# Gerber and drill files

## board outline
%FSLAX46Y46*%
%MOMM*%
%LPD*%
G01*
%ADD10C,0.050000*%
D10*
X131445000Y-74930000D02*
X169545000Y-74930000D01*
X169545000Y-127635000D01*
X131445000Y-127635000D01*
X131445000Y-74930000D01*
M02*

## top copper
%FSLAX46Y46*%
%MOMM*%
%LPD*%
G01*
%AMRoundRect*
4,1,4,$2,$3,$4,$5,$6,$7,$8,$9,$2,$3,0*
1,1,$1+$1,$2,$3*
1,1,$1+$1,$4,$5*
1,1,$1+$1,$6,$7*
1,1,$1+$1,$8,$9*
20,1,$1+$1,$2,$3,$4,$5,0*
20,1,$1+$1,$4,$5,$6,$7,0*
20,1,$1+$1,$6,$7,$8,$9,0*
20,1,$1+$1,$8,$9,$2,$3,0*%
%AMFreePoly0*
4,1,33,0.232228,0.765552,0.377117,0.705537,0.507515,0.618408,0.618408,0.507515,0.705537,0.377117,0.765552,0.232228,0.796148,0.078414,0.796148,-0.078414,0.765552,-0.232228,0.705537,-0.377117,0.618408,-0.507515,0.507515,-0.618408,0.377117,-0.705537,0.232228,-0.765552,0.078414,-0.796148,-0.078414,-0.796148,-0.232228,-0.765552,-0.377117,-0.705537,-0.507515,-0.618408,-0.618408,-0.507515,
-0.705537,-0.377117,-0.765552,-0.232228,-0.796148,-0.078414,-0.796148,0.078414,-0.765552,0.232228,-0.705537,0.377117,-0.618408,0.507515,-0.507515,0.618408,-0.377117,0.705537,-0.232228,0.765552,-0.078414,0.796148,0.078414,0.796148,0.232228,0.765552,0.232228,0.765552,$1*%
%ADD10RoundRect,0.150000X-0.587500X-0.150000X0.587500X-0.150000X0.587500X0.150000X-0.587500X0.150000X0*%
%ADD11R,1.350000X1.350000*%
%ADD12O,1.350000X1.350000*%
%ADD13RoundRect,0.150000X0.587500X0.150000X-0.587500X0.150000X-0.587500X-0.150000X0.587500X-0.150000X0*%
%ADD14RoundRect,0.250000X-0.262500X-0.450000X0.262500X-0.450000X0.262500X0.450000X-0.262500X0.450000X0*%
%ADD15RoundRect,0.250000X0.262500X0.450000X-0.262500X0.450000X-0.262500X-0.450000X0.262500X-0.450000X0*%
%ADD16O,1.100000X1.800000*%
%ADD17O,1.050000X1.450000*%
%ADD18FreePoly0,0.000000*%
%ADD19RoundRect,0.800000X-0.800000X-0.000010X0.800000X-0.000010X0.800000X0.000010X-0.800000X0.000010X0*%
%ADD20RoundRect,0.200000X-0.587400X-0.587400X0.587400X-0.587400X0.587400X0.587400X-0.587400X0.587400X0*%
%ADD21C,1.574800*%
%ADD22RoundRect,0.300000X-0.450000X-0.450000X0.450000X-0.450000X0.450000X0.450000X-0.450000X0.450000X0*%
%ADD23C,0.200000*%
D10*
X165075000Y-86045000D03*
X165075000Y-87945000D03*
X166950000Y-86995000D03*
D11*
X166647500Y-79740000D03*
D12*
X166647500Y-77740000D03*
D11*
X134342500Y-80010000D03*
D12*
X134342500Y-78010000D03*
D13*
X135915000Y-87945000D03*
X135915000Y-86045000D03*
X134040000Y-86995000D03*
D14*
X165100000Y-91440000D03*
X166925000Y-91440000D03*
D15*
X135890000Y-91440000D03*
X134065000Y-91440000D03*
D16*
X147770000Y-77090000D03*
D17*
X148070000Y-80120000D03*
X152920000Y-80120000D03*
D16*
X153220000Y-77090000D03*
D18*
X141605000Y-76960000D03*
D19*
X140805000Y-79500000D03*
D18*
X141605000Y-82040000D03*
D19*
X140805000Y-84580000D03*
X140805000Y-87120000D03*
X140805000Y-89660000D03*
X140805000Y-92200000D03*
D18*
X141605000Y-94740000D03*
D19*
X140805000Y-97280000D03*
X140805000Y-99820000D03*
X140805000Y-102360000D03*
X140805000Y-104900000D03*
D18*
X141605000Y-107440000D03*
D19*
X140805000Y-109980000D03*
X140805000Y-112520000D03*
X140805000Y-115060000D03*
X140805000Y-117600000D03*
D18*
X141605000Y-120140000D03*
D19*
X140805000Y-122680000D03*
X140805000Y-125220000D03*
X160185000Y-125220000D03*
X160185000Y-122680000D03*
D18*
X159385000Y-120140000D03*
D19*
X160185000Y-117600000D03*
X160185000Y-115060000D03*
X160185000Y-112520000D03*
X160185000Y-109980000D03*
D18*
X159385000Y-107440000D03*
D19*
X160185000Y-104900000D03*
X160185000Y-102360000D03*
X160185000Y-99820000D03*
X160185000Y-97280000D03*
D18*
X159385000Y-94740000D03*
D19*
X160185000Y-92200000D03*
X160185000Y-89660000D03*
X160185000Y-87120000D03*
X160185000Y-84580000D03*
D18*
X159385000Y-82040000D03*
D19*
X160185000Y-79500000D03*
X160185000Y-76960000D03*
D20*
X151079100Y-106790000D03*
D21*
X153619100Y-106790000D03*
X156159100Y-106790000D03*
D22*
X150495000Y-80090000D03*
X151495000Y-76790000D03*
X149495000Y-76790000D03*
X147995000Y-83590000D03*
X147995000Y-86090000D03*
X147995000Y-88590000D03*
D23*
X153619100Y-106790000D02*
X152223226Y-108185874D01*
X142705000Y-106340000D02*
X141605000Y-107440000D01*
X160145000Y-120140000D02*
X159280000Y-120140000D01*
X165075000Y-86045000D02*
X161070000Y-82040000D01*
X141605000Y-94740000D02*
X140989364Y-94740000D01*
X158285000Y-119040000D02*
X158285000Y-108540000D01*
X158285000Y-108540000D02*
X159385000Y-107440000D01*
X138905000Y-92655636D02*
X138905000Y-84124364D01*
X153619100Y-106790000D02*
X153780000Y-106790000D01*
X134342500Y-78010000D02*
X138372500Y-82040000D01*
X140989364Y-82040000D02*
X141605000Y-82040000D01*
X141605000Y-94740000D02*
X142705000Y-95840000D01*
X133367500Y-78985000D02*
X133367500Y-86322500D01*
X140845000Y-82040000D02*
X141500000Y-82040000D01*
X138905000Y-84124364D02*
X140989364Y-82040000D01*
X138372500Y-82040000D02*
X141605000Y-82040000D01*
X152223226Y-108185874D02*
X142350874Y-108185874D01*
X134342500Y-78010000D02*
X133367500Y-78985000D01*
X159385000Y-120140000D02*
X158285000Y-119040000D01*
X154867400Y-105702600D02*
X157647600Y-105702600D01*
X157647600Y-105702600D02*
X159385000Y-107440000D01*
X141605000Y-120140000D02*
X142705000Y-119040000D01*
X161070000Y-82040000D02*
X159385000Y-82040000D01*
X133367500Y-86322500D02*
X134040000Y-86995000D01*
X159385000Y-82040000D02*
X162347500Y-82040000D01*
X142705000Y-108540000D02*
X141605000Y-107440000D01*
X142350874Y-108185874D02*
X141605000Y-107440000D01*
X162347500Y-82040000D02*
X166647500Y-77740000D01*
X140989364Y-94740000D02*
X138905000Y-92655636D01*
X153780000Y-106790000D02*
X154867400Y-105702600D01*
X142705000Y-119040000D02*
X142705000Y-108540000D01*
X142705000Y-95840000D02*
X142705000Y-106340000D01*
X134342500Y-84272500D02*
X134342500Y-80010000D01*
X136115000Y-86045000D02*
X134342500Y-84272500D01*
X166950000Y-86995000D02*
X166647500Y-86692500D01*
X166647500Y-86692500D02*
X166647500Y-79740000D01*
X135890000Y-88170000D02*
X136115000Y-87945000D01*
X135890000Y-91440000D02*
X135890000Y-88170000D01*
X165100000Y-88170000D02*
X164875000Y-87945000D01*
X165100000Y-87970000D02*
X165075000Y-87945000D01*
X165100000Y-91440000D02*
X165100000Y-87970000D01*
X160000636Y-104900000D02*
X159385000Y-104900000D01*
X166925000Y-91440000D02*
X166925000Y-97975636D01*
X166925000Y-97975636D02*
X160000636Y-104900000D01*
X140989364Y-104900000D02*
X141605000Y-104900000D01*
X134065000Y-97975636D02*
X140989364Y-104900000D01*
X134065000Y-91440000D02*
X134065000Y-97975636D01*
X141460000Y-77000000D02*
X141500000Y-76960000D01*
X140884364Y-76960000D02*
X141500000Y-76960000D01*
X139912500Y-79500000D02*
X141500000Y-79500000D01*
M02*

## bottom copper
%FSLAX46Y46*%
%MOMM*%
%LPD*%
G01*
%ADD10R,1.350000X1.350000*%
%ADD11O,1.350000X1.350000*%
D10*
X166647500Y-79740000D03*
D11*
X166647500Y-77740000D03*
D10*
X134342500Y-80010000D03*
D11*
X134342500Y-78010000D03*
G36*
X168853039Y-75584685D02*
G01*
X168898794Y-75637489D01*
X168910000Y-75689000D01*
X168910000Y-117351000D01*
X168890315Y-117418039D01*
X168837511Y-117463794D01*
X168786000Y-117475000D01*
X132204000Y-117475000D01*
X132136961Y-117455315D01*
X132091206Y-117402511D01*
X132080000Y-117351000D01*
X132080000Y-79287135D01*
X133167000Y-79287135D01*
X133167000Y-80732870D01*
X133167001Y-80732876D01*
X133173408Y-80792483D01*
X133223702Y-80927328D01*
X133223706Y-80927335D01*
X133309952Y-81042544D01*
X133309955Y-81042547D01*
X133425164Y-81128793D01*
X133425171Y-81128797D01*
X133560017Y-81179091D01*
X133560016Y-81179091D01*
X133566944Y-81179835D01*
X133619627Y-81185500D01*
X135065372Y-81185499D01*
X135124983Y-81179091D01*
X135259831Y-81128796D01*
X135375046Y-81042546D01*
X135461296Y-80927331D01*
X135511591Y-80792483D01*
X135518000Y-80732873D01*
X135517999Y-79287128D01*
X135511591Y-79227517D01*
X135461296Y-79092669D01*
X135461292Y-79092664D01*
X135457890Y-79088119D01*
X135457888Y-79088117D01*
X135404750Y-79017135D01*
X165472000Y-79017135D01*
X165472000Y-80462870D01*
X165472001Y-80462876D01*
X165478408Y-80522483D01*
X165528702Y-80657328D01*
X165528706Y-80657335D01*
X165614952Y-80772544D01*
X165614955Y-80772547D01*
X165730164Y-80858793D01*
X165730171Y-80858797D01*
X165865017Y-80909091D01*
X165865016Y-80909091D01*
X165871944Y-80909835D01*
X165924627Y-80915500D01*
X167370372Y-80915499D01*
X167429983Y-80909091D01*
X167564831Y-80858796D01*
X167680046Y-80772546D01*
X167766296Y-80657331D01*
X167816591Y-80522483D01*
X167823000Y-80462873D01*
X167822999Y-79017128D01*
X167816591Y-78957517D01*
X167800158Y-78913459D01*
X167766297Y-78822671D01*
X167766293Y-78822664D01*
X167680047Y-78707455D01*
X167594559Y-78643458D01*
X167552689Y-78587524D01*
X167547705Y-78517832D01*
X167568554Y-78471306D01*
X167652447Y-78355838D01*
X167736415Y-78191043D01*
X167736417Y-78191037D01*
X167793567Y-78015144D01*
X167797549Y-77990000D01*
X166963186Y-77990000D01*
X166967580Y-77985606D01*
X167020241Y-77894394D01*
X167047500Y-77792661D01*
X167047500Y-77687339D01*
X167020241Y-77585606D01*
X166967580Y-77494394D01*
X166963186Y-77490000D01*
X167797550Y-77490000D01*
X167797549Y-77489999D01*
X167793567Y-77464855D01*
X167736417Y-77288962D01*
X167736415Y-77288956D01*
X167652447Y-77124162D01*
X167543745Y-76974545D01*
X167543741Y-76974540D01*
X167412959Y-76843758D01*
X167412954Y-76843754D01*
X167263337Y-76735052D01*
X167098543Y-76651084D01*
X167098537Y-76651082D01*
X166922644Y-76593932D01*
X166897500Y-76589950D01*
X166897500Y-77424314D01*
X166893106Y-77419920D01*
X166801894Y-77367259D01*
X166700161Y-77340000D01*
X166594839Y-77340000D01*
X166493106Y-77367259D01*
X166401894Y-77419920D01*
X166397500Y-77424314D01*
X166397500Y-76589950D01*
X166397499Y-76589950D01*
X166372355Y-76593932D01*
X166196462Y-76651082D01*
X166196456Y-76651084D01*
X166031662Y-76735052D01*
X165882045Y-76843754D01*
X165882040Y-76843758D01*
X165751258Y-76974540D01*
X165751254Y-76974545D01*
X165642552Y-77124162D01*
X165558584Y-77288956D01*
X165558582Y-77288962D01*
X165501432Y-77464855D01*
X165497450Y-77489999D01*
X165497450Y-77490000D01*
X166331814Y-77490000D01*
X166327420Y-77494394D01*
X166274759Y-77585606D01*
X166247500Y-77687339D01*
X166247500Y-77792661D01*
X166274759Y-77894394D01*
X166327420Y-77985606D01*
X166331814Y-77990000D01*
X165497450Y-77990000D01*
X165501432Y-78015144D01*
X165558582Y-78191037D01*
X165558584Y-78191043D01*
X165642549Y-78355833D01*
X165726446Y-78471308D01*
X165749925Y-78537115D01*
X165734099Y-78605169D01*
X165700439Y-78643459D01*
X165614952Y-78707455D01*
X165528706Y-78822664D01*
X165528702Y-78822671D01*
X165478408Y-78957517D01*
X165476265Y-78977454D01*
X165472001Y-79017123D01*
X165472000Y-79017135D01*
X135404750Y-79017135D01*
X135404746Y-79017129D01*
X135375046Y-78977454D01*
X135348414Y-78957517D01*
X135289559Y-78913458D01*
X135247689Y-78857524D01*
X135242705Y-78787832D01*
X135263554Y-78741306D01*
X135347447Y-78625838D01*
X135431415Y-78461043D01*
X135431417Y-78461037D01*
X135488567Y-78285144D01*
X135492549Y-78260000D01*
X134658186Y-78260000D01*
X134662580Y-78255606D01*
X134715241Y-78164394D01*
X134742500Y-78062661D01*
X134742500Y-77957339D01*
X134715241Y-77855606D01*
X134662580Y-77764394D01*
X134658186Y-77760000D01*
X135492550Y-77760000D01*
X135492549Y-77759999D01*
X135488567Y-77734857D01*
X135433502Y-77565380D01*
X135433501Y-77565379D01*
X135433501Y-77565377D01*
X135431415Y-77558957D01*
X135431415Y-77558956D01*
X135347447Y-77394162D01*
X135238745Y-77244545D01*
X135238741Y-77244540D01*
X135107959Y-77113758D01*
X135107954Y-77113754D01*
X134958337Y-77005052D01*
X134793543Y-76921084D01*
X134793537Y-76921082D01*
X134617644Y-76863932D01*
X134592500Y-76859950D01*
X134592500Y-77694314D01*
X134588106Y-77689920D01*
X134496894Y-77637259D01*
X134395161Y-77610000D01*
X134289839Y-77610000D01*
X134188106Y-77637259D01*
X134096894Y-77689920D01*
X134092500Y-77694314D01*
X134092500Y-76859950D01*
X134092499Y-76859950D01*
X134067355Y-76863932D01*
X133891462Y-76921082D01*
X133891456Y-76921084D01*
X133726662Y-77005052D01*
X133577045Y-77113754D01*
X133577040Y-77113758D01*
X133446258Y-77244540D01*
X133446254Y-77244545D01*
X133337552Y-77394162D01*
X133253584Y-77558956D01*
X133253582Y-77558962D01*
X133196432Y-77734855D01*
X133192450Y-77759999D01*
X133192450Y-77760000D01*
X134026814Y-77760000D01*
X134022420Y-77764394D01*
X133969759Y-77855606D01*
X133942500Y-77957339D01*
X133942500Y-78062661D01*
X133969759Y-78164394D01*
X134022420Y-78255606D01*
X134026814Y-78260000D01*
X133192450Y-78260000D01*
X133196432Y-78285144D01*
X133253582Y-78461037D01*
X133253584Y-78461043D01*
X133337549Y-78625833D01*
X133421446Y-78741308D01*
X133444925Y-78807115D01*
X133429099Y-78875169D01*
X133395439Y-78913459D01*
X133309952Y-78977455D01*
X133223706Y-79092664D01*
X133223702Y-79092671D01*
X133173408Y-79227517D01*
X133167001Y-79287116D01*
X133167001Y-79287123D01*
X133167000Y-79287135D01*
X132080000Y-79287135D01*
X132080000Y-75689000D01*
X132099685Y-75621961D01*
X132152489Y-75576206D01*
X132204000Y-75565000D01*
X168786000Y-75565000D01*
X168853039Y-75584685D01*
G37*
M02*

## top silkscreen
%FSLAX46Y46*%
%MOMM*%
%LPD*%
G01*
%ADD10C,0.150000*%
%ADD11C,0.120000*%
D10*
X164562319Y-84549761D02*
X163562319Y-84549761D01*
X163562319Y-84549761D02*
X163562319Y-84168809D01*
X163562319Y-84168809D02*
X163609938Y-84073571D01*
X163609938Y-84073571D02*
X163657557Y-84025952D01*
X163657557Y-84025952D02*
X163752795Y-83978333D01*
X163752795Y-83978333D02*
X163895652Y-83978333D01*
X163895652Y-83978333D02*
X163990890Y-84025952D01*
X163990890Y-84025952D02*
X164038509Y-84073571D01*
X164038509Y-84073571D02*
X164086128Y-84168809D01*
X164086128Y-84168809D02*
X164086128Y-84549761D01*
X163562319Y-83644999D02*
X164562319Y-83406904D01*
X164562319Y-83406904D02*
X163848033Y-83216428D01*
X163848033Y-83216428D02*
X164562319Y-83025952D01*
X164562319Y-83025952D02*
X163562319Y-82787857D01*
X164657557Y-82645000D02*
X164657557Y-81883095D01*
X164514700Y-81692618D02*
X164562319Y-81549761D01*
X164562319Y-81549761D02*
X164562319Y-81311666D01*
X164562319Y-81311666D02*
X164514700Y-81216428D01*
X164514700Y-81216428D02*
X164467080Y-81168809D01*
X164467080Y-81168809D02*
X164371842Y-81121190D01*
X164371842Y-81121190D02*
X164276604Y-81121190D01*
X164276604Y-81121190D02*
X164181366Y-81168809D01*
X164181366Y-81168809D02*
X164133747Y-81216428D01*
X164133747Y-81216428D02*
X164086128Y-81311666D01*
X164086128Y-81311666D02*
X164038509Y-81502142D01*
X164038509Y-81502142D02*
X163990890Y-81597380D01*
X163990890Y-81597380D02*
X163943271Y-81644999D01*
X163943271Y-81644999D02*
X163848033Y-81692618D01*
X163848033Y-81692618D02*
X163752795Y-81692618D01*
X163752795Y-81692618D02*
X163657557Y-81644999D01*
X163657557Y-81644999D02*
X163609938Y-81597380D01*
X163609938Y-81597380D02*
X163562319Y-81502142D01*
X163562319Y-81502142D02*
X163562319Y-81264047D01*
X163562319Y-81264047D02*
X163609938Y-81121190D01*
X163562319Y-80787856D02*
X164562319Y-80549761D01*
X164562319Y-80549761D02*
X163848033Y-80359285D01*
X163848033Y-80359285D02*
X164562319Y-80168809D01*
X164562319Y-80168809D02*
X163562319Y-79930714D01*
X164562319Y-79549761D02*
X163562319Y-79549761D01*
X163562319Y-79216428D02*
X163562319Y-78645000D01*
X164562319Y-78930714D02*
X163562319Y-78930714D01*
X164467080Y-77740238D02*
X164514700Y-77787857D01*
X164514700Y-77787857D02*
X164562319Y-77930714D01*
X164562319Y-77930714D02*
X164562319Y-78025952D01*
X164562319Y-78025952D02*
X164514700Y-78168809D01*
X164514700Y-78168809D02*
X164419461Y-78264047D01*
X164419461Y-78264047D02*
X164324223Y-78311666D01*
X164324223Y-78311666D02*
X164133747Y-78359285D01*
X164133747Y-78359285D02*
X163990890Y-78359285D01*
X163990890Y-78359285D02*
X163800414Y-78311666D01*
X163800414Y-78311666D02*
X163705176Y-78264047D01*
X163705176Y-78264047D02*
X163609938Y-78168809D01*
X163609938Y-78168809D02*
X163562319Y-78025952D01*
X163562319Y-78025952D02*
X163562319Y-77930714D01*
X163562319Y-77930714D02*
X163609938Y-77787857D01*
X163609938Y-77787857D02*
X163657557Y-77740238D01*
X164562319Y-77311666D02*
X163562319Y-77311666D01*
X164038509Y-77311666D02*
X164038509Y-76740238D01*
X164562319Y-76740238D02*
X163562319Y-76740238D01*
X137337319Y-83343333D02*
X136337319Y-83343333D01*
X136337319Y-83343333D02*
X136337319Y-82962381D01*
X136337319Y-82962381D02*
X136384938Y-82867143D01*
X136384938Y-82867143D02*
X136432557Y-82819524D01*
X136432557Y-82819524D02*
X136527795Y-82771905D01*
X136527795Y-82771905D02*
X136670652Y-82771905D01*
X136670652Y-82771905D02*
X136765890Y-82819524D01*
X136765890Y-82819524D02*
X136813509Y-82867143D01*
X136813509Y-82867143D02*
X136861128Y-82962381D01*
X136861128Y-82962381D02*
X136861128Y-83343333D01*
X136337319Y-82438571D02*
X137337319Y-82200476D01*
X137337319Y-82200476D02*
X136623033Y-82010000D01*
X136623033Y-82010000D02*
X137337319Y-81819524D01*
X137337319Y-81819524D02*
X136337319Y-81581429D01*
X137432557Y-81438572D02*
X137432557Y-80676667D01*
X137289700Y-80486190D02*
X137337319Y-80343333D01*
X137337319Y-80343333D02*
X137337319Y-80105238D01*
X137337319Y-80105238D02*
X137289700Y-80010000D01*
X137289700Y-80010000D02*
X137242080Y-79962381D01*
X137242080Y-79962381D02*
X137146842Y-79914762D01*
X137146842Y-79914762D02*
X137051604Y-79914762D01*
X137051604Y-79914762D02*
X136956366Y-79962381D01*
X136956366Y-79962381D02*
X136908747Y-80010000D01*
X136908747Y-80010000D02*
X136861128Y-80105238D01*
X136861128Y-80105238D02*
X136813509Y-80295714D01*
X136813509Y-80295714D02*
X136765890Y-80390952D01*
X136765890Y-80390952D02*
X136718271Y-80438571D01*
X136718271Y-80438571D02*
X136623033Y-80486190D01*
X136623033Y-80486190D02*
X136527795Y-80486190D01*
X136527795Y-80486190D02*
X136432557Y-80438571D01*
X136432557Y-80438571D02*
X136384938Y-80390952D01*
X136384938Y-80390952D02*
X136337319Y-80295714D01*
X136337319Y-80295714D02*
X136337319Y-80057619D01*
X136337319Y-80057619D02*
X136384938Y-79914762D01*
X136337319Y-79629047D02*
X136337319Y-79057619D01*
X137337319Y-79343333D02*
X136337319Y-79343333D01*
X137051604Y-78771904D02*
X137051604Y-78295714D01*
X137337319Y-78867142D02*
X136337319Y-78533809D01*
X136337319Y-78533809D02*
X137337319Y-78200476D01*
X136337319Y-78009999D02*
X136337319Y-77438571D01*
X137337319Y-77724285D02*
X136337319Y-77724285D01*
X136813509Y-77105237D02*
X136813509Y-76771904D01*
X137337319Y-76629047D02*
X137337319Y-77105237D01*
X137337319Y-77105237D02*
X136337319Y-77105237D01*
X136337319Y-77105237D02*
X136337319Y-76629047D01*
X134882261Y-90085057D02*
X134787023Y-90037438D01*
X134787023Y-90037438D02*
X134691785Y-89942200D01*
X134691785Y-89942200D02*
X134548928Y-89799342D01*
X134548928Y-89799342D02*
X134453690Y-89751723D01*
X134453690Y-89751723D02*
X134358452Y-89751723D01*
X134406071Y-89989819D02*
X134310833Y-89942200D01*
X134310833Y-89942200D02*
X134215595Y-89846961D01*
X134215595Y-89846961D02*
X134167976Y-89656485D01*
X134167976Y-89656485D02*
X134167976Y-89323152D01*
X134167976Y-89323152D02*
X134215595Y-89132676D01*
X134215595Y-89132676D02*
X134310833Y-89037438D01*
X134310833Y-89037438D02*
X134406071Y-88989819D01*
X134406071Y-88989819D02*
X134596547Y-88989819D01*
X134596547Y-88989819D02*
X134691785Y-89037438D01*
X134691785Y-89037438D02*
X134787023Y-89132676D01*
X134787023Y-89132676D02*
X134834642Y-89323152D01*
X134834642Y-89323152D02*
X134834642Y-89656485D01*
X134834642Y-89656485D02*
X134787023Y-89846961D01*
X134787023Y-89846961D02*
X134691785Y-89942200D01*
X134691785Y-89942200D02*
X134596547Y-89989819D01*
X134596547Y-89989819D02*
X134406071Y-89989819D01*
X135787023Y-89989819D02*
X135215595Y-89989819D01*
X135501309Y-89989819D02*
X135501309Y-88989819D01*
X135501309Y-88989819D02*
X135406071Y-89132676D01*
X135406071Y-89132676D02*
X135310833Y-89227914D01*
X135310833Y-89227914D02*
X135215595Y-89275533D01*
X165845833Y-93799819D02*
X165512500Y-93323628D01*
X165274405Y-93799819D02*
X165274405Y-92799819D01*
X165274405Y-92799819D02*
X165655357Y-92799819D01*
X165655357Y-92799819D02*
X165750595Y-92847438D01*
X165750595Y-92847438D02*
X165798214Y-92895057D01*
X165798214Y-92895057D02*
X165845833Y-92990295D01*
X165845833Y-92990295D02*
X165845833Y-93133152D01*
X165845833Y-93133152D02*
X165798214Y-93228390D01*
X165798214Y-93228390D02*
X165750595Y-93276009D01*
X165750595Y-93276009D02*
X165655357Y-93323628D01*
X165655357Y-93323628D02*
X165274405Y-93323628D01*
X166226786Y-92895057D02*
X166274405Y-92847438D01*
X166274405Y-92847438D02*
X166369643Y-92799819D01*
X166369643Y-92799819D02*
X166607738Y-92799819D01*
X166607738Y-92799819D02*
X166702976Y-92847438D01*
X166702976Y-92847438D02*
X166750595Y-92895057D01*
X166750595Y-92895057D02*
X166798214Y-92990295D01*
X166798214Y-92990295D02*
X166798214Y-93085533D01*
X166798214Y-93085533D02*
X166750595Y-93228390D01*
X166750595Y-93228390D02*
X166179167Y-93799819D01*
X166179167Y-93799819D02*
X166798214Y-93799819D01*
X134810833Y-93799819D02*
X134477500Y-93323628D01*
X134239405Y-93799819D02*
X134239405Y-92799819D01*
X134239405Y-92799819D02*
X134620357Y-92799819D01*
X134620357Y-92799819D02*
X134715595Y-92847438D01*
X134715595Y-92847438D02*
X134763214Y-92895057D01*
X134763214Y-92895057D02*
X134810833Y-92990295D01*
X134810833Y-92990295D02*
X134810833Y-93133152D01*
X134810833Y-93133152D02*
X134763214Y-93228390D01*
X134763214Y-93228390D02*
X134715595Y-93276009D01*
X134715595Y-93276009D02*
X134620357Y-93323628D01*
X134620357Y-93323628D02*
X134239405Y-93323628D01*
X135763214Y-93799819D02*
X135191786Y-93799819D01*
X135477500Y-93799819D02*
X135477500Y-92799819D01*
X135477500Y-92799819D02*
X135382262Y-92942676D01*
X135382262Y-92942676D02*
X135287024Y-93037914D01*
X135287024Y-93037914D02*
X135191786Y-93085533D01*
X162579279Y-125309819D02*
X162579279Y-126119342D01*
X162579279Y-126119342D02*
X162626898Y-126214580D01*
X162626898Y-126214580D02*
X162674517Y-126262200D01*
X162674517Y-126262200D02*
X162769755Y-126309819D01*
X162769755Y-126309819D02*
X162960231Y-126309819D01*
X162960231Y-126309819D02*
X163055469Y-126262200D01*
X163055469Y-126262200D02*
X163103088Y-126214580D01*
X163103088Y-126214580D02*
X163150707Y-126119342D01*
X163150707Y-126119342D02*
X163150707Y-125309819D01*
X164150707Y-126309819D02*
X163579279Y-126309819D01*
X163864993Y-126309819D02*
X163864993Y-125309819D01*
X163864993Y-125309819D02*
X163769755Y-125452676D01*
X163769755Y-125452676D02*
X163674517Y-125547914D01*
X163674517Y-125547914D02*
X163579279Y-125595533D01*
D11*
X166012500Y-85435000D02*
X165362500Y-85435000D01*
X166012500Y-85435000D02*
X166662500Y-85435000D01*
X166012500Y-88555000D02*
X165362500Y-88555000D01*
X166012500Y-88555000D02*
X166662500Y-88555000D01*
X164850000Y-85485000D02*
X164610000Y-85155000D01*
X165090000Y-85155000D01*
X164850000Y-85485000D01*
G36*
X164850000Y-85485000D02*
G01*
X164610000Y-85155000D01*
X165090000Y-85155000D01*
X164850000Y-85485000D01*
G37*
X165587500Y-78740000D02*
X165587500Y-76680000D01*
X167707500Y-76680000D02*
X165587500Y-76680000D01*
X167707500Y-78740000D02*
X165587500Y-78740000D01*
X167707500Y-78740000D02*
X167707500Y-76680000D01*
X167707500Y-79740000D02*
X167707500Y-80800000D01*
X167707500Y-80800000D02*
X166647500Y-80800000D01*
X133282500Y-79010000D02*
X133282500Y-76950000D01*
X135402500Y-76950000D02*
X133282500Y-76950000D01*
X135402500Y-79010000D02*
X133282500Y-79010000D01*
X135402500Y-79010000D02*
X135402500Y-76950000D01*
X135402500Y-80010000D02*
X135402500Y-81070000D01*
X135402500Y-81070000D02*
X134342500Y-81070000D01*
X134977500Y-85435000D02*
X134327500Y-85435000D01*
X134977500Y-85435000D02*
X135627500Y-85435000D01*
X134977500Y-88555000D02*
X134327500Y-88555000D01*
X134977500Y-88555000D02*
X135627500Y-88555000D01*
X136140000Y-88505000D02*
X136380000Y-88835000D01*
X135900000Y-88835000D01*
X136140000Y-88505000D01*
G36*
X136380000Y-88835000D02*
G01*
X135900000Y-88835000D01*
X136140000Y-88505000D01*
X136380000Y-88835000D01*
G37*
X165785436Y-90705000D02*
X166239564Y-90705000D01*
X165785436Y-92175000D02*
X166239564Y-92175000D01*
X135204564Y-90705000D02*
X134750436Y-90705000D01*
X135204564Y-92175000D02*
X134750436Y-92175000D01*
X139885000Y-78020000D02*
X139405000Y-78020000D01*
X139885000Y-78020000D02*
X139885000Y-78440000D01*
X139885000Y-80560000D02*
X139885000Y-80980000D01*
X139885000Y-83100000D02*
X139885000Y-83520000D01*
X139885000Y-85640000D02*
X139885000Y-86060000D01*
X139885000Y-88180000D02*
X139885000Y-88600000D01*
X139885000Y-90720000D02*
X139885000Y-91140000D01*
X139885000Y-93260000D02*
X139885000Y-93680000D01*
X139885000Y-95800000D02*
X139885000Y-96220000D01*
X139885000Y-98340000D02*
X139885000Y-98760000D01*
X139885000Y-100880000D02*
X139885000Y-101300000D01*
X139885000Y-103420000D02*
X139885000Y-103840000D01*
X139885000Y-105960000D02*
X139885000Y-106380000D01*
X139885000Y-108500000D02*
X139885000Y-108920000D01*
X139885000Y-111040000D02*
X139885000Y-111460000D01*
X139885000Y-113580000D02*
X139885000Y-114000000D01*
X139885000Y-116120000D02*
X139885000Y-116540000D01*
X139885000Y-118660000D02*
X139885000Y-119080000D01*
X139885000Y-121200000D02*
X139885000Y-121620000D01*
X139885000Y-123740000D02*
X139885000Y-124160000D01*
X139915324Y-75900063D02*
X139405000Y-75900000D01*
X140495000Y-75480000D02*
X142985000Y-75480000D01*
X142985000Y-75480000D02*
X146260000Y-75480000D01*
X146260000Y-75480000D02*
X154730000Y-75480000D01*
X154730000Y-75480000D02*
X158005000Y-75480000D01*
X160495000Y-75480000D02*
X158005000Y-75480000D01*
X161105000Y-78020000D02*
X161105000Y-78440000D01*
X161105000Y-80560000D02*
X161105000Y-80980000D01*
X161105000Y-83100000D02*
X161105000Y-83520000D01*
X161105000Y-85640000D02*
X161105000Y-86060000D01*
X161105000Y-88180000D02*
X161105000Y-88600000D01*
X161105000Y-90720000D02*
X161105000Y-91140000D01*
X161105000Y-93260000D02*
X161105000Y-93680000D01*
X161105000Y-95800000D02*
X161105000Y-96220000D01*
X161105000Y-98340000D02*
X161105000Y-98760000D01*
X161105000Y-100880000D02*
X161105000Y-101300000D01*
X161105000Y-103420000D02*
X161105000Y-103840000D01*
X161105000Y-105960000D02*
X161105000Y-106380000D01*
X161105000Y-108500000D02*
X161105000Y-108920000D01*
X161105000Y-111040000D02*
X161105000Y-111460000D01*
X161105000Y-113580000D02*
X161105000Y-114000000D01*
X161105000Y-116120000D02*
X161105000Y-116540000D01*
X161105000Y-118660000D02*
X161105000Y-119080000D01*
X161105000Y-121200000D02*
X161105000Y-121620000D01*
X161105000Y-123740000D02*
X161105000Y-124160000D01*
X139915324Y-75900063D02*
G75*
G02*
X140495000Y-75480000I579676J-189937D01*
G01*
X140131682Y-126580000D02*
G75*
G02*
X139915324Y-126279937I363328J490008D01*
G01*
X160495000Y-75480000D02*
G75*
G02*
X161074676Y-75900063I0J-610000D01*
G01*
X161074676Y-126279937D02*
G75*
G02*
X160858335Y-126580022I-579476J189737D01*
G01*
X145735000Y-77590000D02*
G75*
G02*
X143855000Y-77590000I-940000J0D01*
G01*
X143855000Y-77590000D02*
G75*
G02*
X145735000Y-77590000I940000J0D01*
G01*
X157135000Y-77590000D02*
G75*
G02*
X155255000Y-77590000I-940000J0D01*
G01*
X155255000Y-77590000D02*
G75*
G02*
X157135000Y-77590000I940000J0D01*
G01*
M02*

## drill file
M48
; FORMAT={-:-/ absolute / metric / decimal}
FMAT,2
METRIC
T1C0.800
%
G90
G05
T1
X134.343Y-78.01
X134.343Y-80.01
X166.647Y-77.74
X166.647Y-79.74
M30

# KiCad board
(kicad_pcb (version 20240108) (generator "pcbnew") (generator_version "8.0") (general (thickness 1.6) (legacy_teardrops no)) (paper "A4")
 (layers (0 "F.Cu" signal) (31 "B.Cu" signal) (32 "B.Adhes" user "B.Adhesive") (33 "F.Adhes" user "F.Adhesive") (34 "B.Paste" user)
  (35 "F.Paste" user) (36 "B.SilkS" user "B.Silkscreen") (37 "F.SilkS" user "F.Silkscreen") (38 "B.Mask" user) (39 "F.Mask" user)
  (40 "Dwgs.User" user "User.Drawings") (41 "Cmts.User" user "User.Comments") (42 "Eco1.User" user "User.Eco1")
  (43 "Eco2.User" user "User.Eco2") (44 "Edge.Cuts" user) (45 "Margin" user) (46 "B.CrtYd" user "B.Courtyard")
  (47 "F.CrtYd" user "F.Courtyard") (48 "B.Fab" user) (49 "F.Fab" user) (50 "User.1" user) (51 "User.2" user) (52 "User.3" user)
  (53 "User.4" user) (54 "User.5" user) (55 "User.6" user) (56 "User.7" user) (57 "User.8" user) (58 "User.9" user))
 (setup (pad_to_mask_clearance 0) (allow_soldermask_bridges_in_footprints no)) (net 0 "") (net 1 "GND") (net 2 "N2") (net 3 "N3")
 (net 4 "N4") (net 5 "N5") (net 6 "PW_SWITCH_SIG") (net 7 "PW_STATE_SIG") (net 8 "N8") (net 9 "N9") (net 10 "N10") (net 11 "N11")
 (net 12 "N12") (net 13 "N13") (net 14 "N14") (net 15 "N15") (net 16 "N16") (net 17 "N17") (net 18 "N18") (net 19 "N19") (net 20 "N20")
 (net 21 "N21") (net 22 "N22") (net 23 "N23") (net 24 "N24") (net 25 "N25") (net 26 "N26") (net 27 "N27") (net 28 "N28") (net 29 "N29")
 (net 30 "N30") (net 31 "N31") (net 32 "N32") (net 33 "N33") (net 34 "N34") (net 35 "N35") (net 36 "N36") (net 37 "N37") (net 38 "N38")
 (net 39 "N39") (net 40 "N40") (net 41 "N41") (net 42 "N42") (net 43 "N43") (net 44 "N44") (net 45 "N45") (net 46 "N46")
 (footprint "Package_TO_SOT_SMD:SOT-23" (layer "F.Cu") (at 166.0125 86.995)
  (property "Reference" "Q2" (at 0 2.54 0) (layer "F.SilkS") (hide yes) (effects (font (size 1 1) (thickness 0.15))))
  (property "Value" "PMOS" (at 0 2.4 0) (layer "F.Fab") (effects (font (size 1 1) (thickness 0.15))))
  (fp_line (start 0 -1.56) (end -0.65 -1.56) (stroke (width 0.12) (type solid)) (layer "F.SilkS"))
  (fp_line (start 0 -1.56) (end 0.65 -1.56) (stroke (width 0.12) (type solid)) (layer "F.SilkS"))
  (fp_line (start 0 1.56) (end -0.65 1.56) (stroke (width 0.12) (type solid)) (layer "F.SilkS"))
  (fp_line (start 0 1.56) (end 0.65 1.56) (stroke (width 0.12) (type solid)) (layer "F.SilkS"))
  (fp_poly
   (pts (xy -1.1625 -1.51) (xy -1.4025 -1.84) (xy -0.9225 -1.84) (xy -1.1625 -1.51)) (stroke (width 0.12) (type solid)) (fill solid)
   (layer "F.SilkS"))
  (pad "1" smd roundrect (at -0.9375 -0.95) (size 1.475 0.6) (layers "F.Cu" "F.Paste" "F.Mask") (roundrect_rratio 0.25) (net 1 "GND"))
  (pad "2" smd roundrect (at -0.9375 0.95) (size 1.475 0.6) (layers "F.Cu" "F.Paste" "F.Mask") (roundrect_rratio 0.25) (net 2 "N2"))
  (pad "3" smd roundrect (at 0.9375 0) (size 1.475 0.6) (layers "F.Cu" "F.Paste" "F.Mask") (roundrect_rratio 0.25) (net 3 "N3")))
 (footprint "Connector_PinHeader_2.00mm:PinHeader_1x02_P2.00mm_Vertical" (layer "F.Cu") (at 166.6475 79.74 180)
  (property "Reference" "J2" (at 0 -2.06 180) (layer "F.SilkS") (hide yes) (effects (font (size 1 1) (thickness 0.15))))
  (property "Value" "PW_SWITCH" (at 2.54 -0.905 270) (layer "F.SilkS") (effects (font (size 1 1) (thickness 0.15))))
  (fp_line (start 1.06 1) (end 1.06 3.06) (stroke (width 0.12) (type solid)) (layer "F.SilkS"))
  (fp_line (start -1.06 3.06) (end 1.06 3.06) (stroke (width 0.12) (type solid)) (layer "F.SilkS"))
  (fp_line (start -1.06 1) (end 1.06 1) (stroke (width 0.12) (type solid)) (layer "F.SilkS"))
  (fp_line (start -1.06 1) (end -1.06 3.06) (stroke (width 0.12) (type solid)) (layer "F.SilkS"))
  (fp_line (start -1.06 0) (end -1.06 -1.06) (stroke (width 0.12) (type solid)) (layer "F.SilkS"))
  (fp_line (start -1.06 -1.06) (end 0 -1.06) (stroke (width 0.12) (type solid)) (layer "F.SilkS"))
  (pad "1" thru_hole rect (at 0 0 180) (size 1.35 1.35) (drill 0.8) (layers "*.Cu" "*.Mask") (remove_unused_layers no) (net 3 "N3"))
  (pad "2" thru_hole oval (at 0 2 180) (size 1.35 1.35) (drill 0.8) (layers "*.Cu" "*.Mask") (remove_unused_layers no) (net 1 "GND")))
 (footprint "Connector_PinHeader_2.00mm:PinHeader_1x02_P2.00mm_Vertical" (layer "F.Cu") (at 134.3425 80.01 180)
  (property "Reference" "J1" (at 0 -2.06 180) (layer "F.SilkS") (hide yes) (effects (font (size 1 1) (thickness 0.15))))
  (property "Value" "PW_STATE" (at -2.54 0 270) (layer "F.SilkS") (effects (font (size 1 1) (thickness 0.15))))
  (fp_line (start 1.06 1) (end 1.06 3.06) (stroke (width 0.12) (type solid)) (layer "F.SilkS"))
  (fp_line (start -1.06 3.06) (end 1.06 3.06) (stroke (width 0.12) (type solid)) (layer "F.SilkS"))
  (fp_line (start -1.06 1) (end 1.06 1) (stroke (width 0.12) (type solid)) (layer "F.SilkS"))
  (fp_line (start -1.06 1) (end -1.06 3.06) (stroke (width 0.12) (type solid)) (layer "F.SilkS"))
  (fp_line (start -1.06 0) (end -1.06 -1.06) (stroke (width 0.12) (type solid)) (layer "F.SilkS"))
  (fp_line (start -1.06 -1.06) (end 0 -1.06) (stroke (width 0.12) (type solid)) (layer "F.SilkS"))
  (pad "1" thru_hole rect (at 0 0 180) (size 1.35 1.35) (drill 0.8) (layers "*.Cu" "*.Mask") (remove_unused_layers no) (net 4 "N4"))
  (pad "2" thru_hole oval (at 0 2 180) (size 1.35 1.35) (drill 0.8) (layers "*.Cu" "*.Mask") (remove_unused_layers no) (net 1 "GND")))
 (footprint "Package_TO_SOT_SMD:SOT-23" (layer "F.Cu") (at 134.9775 86.995 180)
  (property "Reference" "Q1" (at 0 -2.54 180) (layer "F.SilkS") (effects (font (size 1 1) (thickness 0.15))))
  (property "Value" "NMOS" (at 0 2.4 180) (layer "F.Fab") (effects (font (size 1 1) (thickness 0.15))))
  (fp_line (start 0 1.56) (end 0.65 1.56) (stroke (width 0.12) (type solid)) (layer "F.SilkS"))
  (fp_line (start 0 1.56) (end -0.65 1.56) (stroke (width 0.12) (type solid)) (layer "F.SilkS"))
  (fp_line (start 0 -1.56) (end 0.65 -1.56) (stroke (width 0.12) (type solid)) (layer "F.SilkS"))
  (fp_line (start 0 -1.56) (end -0.65 -1.56) (stroke (width 0.12) (type solid)) (layer "F.SilkS"))
  (fp_poly
   (pts (xy -1.1625 -1.51) (xy -1.4025 -1.84) (xy -0.9225 -1.84) (xy -1.1625 -1.51)) (stroke (width 0.12) (type solid)) (fill solid)
   (layer "F.SilkS"))
  (pad "1" smd roundrect (at -0.9375 -0.95 180) (size 1.475 0.6) (layers "F.Cu" "F.Paste" "F.Mask") (roundrect_rratio 0.25) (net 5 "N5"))
  (pad "2" smd roundrect (at -0.9375 0.95 180) (size 1.475 0.6) (layers "F.Cu" "F.Paste" "F.Mask") (roundrect_rratio 0.25) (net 4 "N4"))
  (pad "3" smd roundrect (at 0.9375 0 180) (size 1.475 0.6) (layers "F.Cu" "F.Paste" "F.Mask") (roundrect_rratio 0.25) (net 1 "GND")))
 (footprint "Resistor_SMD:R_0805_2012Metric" (layer "F.Cu") (at 166.0125 91.44)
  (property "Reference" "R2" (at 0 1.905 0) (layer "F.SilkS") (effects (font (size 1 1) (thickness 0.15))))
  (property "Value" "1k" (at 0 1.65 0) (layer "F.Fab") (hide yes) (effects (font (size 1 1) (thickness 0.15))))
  (fp_line (start -0.227064 -0.735) (end 0.227064 -0.735) (stroke (width 0.12) (type solid)) (layer "F.SilkS"))
  (fp_line (start -0.227064 0.735) (end 0.227064 0.735) (stroke (width 0.12) (type solid)) (layer "F.SilkS"))
  (pad "1" smd roundrect (at -0.9125 0) (size 1.025 1.4) (layers "F.Cu" "F.Paste" "F.Mask") (roundrect_rratio 0.243902) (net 2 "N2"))
  (pad "2" smd roundrect (at 0.9125 0) (size 1.025 1.4) (layers "F.Cu" "F.Paste" "F.Mask") (roundrect_rratio 0.243902)
   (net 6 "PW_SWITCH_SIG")))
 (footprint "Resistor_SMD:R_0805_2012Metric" (layer "F.Cu") (at 134.9775 91.44 180)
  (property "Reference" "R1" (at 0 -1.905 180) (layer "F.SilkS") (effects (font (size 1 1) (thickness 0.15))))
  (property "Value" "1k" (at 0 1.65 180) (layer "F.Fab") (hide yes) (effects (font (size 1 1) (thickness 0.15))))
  (fp_line (start -0.227064 0.735) (end 0.227064 0.735) (stroke (width 0.12) (type solid)) (layer "F.SilkS"))
  (fp_line (start -0.227064 -0.735) (end 0.227064 -0.735) (stroke (width 0.12) (type solid)) (layer "F.SilkS"))
  (pad "1" smd roundrect (at -0.9125 0 180) (size 1.025 1.4) (layers "F.Cu" "F.Paste" "F.Mask") (roundrect_rratio 0.243902) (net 5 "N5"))
  (pad "2" smd roundrect (at 0.9125 0 180) (size 1.025 1.4) (layers "F.Cu" "F.Paste" "F.Mask") (roundrect_rratio 0.243902)
   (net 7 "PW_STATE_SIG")))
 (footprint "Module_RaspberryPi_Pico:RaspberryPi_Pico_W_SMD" (layer "F.Cu") (at 150.495 101.09)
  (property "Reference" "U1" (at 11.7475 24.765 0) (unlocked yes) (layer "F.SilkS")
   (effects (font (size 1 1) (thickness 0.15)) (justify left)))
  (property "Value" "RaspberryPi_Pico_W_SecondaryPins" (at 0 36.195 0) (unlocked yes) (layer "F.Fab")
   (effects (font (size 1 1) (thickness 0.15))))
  (fp_line (start -10.61 -23.07) (end -11.09 -23.07) (stroke (width 0.12) (type solid)) (layer "F.SilkS"))
  (fp_line (start -10.61 -23.07) (end -10.61 -22.65) (stroke (width 0.12) (type solid)) (layer "F.SilkS"))
  (fp_line (start -10.61 -20.53) (end -10.61 -20.11) (stroke (width 0.12) (type solid)) (layer "F.SilkS"))
  (fp_line (start -10.61 -17.99) (end -10.61 -17.57) (stroke (width 0.12) (type solid)) (layer "F.SilkS"))
  (fp_line (start -10.61 -15.45) (end -10.61 -15.03) (stroke (width 0.12) (type solid)) (layer "F.SilkS"))
  (fp_line (start -10.61 -12.91) (end -10.61 -12.49) (stroke (width 0.12) (type solid)) (layer "F.SilkS"))
  (fp_line (start -10.61 -10.37) (end -10.61 -9.95) (stroke (width 0.12) (type solid)) (layer "F.SilkS"))
  (fp_line (start -10.61 -7.83) (end -10.61 -7.41) (stroke (width 0.12) (type solid)) (layer "F.SilkS"))
  (fp_line (start -10.61 -5.29) (end -10.61 -4.87) (stroke (width 0.12) (type solid)) (layer "F.SilkS"))
  (fp_line (start -10.61 -2.75) (end -10.61 -2.33) (stroke (width 0.12) (type solid)) (layer "F.SilkS"))
  (fp_line (start -10.61 -0.21) (end -10.61 0.21) (stroke (width 0.12) (type solid)) (layer "F.SilkS"))
  (fp_line (start -10.61 2.33) (end -10.61 2.75) (stroke (width 0.12) (type solid)) (layer "F.SilkS"))
  (fp_line (start -10.61 4.87) (end -10.61 5.29) (stroke (width 0.12) (type solid)) (layer "F.SilkS"))
  (fp_line (start -10.61 7.41) (end -10.61 7.83) (stroke (width 0.12) (type solid)) (layer "F.SilkS"))
  (fp_line (start -10.61 9.95) (end -10.61 10.37) (stroke (width 0.12) (type solid)) (layer "F.SilkS"))
  (fp_line (start -10.61 12.49) (end -10.61 12.91) (stroke (width 0.12) (type solid)) (layer "F.SilkS"))
  (fp_line (start -10.61 15.03) (end -10.61 15.45) (stroke (width 0.12) (type solid)) (layer "F.SilkS"))
  (fp_line (start -10.61 17.57) (end -10.61 17.99) (stroke (width 0.12) (type solid)) (layer "F.SilkS"))
  (fp_line (start -10.61 20.11) (end -10.61 20.53) (stroke (width 0.12) (type solid)) (layer "F.SilkS"))
  (fp_line (start -10.61 22.65) (end -10.61 23.07) (stroke (width 0.12) (type solid)) (layer "F.SilkS"))
  (fp_line (start -10.579676 -25.189937) (end -11.09 -25.19) (stroke (width 0.12) (type solid)) (layer "F.SilkS"))
  (fp_line (start -10 -25.61) (end -7.51 -25.61) (stroke (width 0.12) (type solid)) (layer "F.SilkS"))
  (fp_line (start -7.51 -25.61) (end -4.235 -25.61) (stroke (width 0.12) (type solid)) (layer "F.SilkS"))
  (fp_line (start -4.235 -25.61) (end 4.235 -25.61) (stroke (width 0.12) (type solid)) (layer "F.SilkS"))
  (fp_line (start 4.235 -25.61) (end 7.51 -25.61) (stroke (width 0.12) (type solid)) (layer "F.SilkS"))
  (fp_line (start 10 -25.61) (end 7.51 -25.61) (stroke (width 0.12) (type solid)) (layer "F.SilkS"))
  (fp_line (start 10.61 -23.07) (end 10.61 -22.65) (stroke (width 0.12) (type solid)) (layer "F.SilkS"))
  (fp_line (start 10.61 -20.53) (end 10.61 -20.11) (stroke (width 0.12) (type solid)) (layer "F.SilkS"))
  (fp_line (start 10.61 -17.99) (end 10.61 -17.57) (stroke (width 0.12) (type solid)) (layer "F.SilkS"))
  (fp_line (start 10.61 -15.45) (end 10.61 -15.03) (stroke (width 0.12) (type solid)) (layer "F.SilkS"))
  (fp_line (start 10.61 -12.91) (end 10.61 -12.49) (stroke (width 0.12) (type solid)) (layer "F.SilkS"))
  (fp_line (start 10.61 -10.37) (end 10.61 -9.95) (stroke (width 0.12) (type solid)) (layer "F.SilkS"))
  (fp_line (start 10.61 -7.83) (end 10.61 -7.41) (stroke (width 0.12) (type solid)) (layer "F.SilkS"))
  (fp_line (start 10.61 -5.29) (end 10.61 -4.87) (stroke (width 0.12) (type solid)) (layer "F.SilkS"))
  (fp_line (start 10.61 -2.75) (end 10.61 -2.33) (stroke (width 0.12) (type solid)) (layer "F.SilkS"))
  (fp_line (start 10.61 -0.21) (end 10.61 0.21) (stroke (width 0.12) (type solid)) (layer "F.SilkS"))
  (fp_line (start 10.61 2.33) (end 10.61 2.75) (stroke (width 0.12) (type solid)) (layer "F.SilkS"))
  (fp_line (start 10.61 4.87) (end 10.61 5.29) (stroke (width 0.12) (type solid)) (layer "F.SilkS"))
  (fp_line (start 10.61 7.41) (end 10.61 7.83) (stroke (width 0.12) (type solid)) (layer "F.SilkS"))
  (fp_line (start 10.61 9.95) (end 10.61 10.37) (stroke (width 0.12) (type solid)) (layer "F.SilkS"))
  (fp_line (start 10.61 12.49) (end 10.61 12.91) (stroke (width 0.12) (type solid)) (layer "F.SilkS"))
  (fp_line (start 10.61 15.03) (end 10.61 15.45) (stroke (width 0.12) (type solid)) (layer "F.SilkS"))
  (fp_line (start 10.61 17.57) (end 10.61 17.99) (stroke (width 0.12) (type solid)) (layer "F.SilkS"))
  (fp_line (start 10.61 20.11) (end 10.61 20.53) (stroke (width 0.12) (type solid)) (layer "F.SilkS"))
  (fp_line (start 10.61 22.65) (end 10.61 23.07) (stroke (width 0.12) (type solid)) (layer "F.SilkS"))
  (fp_arc (start -10.579676 -25.189937) (mid -10.357938 -25.493944) (end -10 -25.61) (stroke (width 0.12) (type solid)) (layer "F.SilkS"))
  (fp_arc (start -10.363318 25.49) (mid -10.494791 25.356765) (end -10.579676 25.189937) (stroke (width 0.12) (type solid))
   (layer "F.SilkS"))
  (fp_arc (start 10 -25.61) (mid 10.357937 -25.493944) (end 10.579676 -25.189937) (stroke (width 0.12) (type solid)) (layer "F.SilkS"))
  (fp_arc (start 10.579676 25.189937) (mid 10.494802 25.356774) (end 10.363318 25.49) (stroke (width 0.12) (type solid)) (layer "F.SilkS"))
  (fp_circle (center -5.7 -23.5) (end -4.76 -23.5) (stroke (width 0.12) (type solid)) (fill none) (layer "F.SilkS"))
  (fp_circle (center 5.7 -23.5) (end 6.64 -23.5) (stroke (width 0.12) (type solid)) (fill none) (layer "F.SilkS"))
  (pad "" smd oval (at -2.725 -24) (size 1.1 1.8) (layers "F.Cu" "F.Paste" "F.Mask"))
  (pad "" smd oval (at -2.425 -20.97) (size 1.05 1.45) (layers "F.Cu" "F.Paste" "F.Mask"))
  (pad "" smd oval (at 2.425 -20.97) (size 1.05 1.45) (layers "F.Cu" "F.Paste" "F.Mask"))
  (pad "" smd oval (at 2.725 -24) (size 1.1 1.8) (layers "F.Cu" "F.Paste" "F.Mask"))
  (pad "1" smd custom (at -8.89 -24.13) (size 1.6 1.6) (layers "F.Cu" "F.Paste" "F.Mask") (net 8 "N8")
   (options (clearance outline) (anchor circle)) (primitives))
  (pad "2" smd roundrect (at -8.89 -21.59) (size 3.2 1.6) (drill (offset -0.8 0)) (layers "F.Cu" "F.Paste" "F.Mask") (roundrect_rratio 0.5)
   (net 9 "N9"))
  (pad "3" smd custom (at -8.89 -19.05) (size 1.6 1.6) (layers "F.Cu" "F.Paste" "F.Mask") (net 1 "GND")
   (options (clearance outline) (anchor circle)) (primitives))
  (pad "4" smd roundrect (at -8.89 -16.51) (size 3.2 1.6) (drill (offset -0.8 0)) (layers "F.Cu" "F.Paste" "F.Mask") (roundrect_rratio 0.5)
   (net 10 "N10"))
  (pad "5" smd roundrect (at -8.89 -13.97) (size 3.2 1.6) (drill (offset -0.8 0)) (layers "F.Cu" "F.Paste" "F.Mask") (roundrect_rratio 0.5)
   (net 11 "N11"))
  (pad "6" smd roundrect (at -8.89 -11.43) (size 3.2 1.6) (drill (offset -0.8 0)) (layers "F.Cu" "F.Paste" "F.Mask") (roundrect_rratio 0.5)
   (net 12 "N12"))
  (pad "7" smd roundrect (at -8.89 -8.89) (size 3.2 1.6) (drill (offset -0.8 0)) (layers "F.Cu" "F.Paste" "F.Mask") (roundrect_rratio 0.5)
   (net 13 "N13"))
  (pad "8" smd custom (at -8.89 -6.35) (size 1.6 1.6) (layers "F.Cu" "F.Paste" "F.Mask") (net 1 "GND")
   (options (clearance outline) (anchor circle)) (primitives))
  (pad "9" smd roundrect (at -8.89 -3.81) (size 3.2 1.6) (drill (offset -0.8 0)) (layers "F.Cu" "F.Paste" "F.Mask") (roundrect_rratio 0.5)
   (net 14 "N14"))
  (pad "10" smd roundrect (at -8.89 -1.27) (size 3.2 1.6) (drill (offset -0.8 0)) (layers "F.Cu" "F.Paste" "F.Mask") (roundrect_rratio 0.5)
   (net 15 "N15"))
  (pad "11" smd roundrect (at -8.89 1.27) (size 3.2 1.6) (drill (offset -0.8 0)) (layers "F.Cu" "F.Paste" "F.Mask") (roundrect_rratio 0.5)
   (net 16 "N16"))
  (pad "12" smd roundrect (at -8.89 3.81) (size 3.2 1.6) (drill (offset -0.8 0)) (layers "F.Cu" "F.Paste" "F.Mask") (roundrect_rratio 0.5)
   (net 7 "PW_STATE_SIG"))
  (pad "13" smd custom (at -8.89 6.35) (size 1.6 1.6) (layers "F.Cu" "F.Paste" "F.Mask") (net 1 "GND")
   (options (clearance outline) (anchor circle)) (primitives))
  (pad "14" smd roundrect (at -8.89 8.89) (size 3.2 1.6) (drill (offset -0.8 0)) (layers "F.Cu" "F.Paste" "F.Mask") (roundrect_rratio 0.5)
   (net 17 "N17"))
  (pad "15" smd roundrect (at -8.89 11.43) (size 3.2 1.6) (drill (offset -0.8 0)) (layers "F.Cu" "F.Paste" "F.Mask") (roundrect_rratio 0.5)
   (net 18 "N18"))
  (pad "16" smd roundrect (at -8.89 13.97) (size 3.2 1.6) (drill (offset -0.8 0)) (layers "F.Cu" "F.Paste" "F.Mask") (roundrect_rratio 0.5)
   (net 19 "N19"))
  (pad "17" smd roundrect (at -8.89 16.51) (size 3.2 1.6) (drill (offset -0.8 0)) (layers "F.Cu" "F.Paste" "F.Mask") (roundrect_rratio 0.5)
   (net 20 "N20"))
  (pad "18" smd custom (at -8.89 19.05) (size 1.6 1.6) (layers "F.Cu" "F.Paste" "F.Mask") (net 1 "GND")
   (options (clearance outline) (anchor circle)) (primitives))
  (pad "19" smd roundrect (at -8.89 21.59) (size 3.2 1.6) (drill (offset -0.8 0)) (layers "F.Cu" "F.Paste" "F.Mask") (roundrect_rratio 0.5)
   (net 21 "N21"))
  (pad "20" smd roundrect (at -8.89 24.13) (size 3.2 1.6) (drill (offset -0.8 0)) (layers "F.Cu" "F.Paste" "F.Mask") (roundrect_rratio 0.5)
   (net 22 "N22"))
  (pad "21" smd roundrect (at 8.89 24.13) (size 3.2 1.6) (drill (offset 0.8 0)) (layers "F.Cu" "F.Paste" "F.Mask") (roundrect_rratio 0.5)
   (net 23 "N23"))
  (pad "22" smd roundrect (at 8.89 21.59) (size 3.2 1.6) (drill (offset 0.8 0)) (layers "F.Cu" "F.Paste" "F.Mask") (roundrect_rratio 0.5)
   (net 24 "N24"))
  (pad "23" smd custom (at 8.89 19.05) (size 1.6 1.6) (layers "F.Cu" "F.Paste" "F.Mask") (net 1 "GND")
   (options (clearance outline) (anchor circle)) (primitives))
  (pad "24" smd roundrect (at 8.89 16.51) (size 3.2 1.6) (drill (offset 0.8 0)) (layers "F.Cu" "F.Paste" "F.Mask") (roundrect_rratio 0.5)
   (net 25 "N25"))
  (pad "25" smd roundrect (at 8.89 13.97) (size 3.2 1.6) (drill (offset 0.8 0)) (layers "F.Cu" "F.Paste" "F.Mask") (roundrect_rratio 0.5)
   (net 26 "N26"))
  (pad "26" smd roundrect (at 8.89 11.43) (size 3.2 1.6) (drill (offset 0.8 0)) (layers "F.Cu" "F.Paste" "F.Mask") (roundrect_rratio 0.5)
   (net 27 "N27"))
  (pad "27" smd roundrect (at 8.89 8.89) (size 3.2 1.6) (drill (offset 0.8 0)) (layers "F.Cu" "F.Paste" "F.Mask") (roundrect_rratio 0.5)
   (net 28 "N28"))
  (pad "28" smd custom (at 8.89 6.35) (size 1.6 1.6) (layers "F.Cu" "F.Paste" "F.Mask") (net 1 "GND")
   (options (clearance outline) (anchor circle)) (primitives))
  (pad "29" smd roundrect (at 8.89 3.81) (size 3.2 1.6) (drill (offset 0.8 0)) (layers "F.Cu" "F.Paste" "F.Mask") (roundrect_rratio 0.5)
   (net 6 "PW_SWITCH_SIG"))
  (pad "30" smd roundrect (at 8.89 1.27) (size 3.2 1.6) (drill (offset 0.8 0)) (layers "F.Cu" "F.Paste" "F.Mask") (roundrect_rratio 0.5)
   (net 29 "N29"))
  (pad "31" smd roundrect (at 8.89 -1.27) (size 3.2 1.6) (drill (offset 0.8 0)) (layers "F.Cu" "F.Paste" "F.Mask") (roundrect_rratio 0.5)
   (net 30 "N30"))
  (pad "32" smd roundrect (at 8.89 -3.81) (size 3.2 1.6) (drill (offset 0.8 0)) (layers "F.Cu" "F.Paste" "F.Mask") (roundrect_rratio 0.5)
   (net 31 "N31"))
  (pad "33" smd custom (at 8.89 -6.35) (size 1.6 1.6) (layers "F.Cu" "F.Paste" "F.Mask") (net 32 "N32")
   (options (clearance outline) (anchor circle)) (primitives))
  (pad "34" smd roundrect (at 8.89 -8.89) (size 3.2 1.6) (drill (offset 0.8 0)) (layers "F.Cu" "F.Paste" "F.Mask") (roundrect_rratio 0.5)
   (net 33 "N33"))
  (pad "35" smd roundrect (at 8.89 -11.43) (size 3.2 1.6) (drill (offset 0.8 0)) (layers "F.Cu" "F.Paste" "F.Mask") (roundrect_rratio 0.5)
   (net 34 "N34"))
  (pad "36" smd roundrect (at 8.89 -13.97) (size 3.2 1.6) (drill (offset 0.8 0)) (layers "F.Cu" "F.Paste" "F.Mask") (roundrect_rratio 0.5)
   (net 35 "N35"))
  (pad "37" smd roundrect (at 8.89 -16.51) (size 3.2 1.6) (drill (offset 0.8 0)) (layers "F.Cu" "F.Paste" "F.Mask") (roundrect_rratio 0.5)
   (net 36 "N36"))
  (pad "38" smd custom (at 8.89 -19.05) (size 1.6 1.6) (layers "F.Cu" "F.Paste" "F.Mask") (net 1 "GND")
   (options (clearance outline) (anchor circle)) (primitives))
  (pad "39" smd roundrect (at 8.89 -21.59) (size 3.2 1.6) (drill (offset 0.8 0)) (layers "F.Cu" "F.Paste" "F.Mask") (roundrect_rratio 0.5)
   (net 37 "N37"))
  (pad "40" smd roundrect (at 8.89 -24.13) (size 3.2 1.6) (drill (offset 0.8 0)) (layers "F.Cu" "F.Paste" "F.Mask") (roundrect_rratio 0.5)
   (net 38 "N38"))
  (pad "D1" smd roundrect (at 0.5841 5.7) (size 1.5748 1.5748) (layers "F.Cu" "F.Paste" "F.Mask") (roundrect_rratio 0.127000254)
   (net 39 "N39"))
  (pad "D2" smd circle (at 3.1241 5.7) (size 1.5748 1.5748) (layers "F.Cu" "F.Paste" "F.Mask") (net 1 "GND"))
  (pad "D3" smd circle (at 5.6641 5.7) (size 1.5748 1.5748) (layers "F.Cu" "F.Paste" "F.Mask") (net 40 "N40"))
  (pad "TP1" smd roundrect (at 0 -21) (size 1.5 1.5) (layers "F.Cu" "F.Paste" "F.Mask") (roundrect_rratio 0.2) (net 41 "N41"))
  (pad "TP2" smd roundrect (at 1 -24.3) (size 1.5 1.5) (layers "F.Cu" "F.Paste" "F.Mask") (roundrect_rratio 0.2) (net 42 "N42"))
  (pad "TP3" smd roundrect (at -1 -24.3) (size 1.5 1.5) (layers "F.Cu" "F.Paste" "F.Mask") (roundrect_rratio 0.2) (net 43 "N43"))
  (pad "TP4" smd roundrect (at -2.5 -17.5) (size 1.5 1.5) (layers "F.Cu" "F.Paste" "F.Mask") (roundrect_rratio 0.2) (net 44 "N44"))
  (pad "TP5" smd roundrect (at -2.5 -15) (size 1.5 1.5) (layers "F.Cu" "F.Paste" "F.Mask") (roundrect_rratio 0.2) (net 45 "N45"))
  (pad "TP6" smd roundrect (at -2.5 -12.5) (size 1.5 1.5) (layers "F.Cu" "F.Paste" "F.Mask") (roundrect_rratio 0.2) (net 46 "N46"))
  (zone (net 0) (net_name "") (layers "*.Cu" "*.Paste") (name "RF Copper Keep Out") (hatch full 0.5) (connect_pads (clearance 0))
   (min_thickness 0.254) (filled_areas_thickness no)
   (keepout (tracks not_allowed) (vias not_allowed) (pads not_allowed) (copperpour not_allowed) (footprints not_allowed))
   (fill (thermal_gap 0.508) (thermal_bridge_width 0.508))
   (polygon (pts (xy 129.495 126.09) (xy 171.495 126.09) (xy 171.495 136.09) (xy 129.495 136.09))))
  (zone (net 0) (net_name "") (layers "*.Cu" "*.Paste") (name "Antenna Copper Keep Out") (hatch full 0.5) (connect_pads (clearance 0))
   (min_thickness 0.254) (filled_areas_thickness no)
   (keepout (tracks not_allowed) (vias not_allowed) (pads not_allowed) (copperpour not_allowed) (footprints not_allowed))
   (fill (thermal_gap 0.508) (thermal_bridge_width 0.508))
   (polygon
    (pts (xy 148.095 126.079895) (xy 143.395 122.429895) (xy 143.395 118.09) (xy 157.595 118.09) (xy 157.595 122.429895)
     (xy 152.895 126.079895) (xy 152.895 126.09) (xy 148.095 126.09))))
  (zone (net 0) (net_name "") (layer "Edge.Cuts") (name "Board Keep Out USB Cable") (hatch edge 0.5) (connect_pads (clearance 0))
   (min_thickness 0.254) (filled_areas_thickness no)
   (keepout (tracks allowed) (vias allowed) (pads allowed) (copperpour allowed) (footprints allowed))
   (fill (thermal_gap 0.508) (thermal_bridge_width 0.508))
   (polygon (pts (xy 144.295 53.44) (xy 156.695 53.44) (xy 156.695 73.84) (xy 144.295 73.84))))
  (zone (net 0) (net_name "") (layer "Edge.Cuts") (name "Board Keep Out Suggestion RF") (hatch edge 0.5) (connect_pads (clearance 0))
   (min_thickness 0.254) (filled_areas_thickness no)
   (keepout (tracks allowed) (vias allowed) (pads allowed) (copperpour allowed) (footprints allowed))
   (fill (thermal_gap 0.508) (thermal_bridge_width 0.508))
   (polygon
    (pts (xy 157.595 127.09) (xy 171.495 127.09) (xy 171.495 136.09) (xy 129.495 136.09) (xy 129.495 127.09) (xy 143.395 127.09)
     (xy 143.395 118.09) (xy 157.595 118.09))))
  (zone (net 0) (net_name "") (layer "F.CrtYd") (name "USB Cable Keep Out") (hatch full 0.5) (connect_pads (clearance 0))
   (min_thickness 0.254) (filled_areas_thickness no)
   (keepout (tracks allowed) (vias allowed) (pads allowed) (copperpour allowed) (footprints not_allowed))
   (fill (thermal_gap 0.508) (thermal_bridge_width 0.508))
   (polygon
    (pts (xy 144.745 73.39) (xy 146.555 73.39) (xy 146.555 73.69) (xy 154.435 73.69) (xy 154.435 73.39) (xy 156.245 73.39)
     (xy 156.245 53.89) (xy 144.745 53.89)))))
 (gr_rect (start 131.445 74.93) (end 169.545 127.635) (stroke (width 0.05) (type default)) (fill none) (layer "Edge.Cuts"))
 (segment (start 153.6191 106.79) (end 152.223226 108.185874) (width 0.2) (layer "F.Cu") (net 1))
 (segment (start 142.705 106.34) (end 141.605 107.44) (width 0.2) (layer "F.Cu") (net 1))
 (segment (start 160.145 120.14) (end 159.28 120.14) (width 0.2) (layer "F.Cu") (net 1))
 (segment (start 165.075 86.045) (end 161.07 82.04) (width 0.2) (layer "F.Cu") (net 1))
 (segment (start 141.605 94.74) (end 140.989364 94.74) (width 0.2) (layer "F.Cu") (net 1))
 (segment (start 158.285 119.04) (end 158.285 108.54) (width 0.2) (layer "F.Cu") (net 1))
 (segment (start 158.285 108.54) (end 159.385 107.44) (width 0.2) (layer "F.Cu") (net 1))
 (segment (start 138.905 92.655636) (end 138.905 84.124364) (width 0.2) (layer "F.Cu") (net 1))
 (segment (start 153.6191 106.79) (end 153.78 106.79) (width 0.2) (layer "F.Cu") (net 1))
 (segment (start 134.3425 78.01) (end 138.3725 82.04) (width 0.2) (layer "F.Cu") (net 1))
 (segment (start 140.989364 82.04) (end 141.605 82.04) (width 0.2) (layer "F.Cu") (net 1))
 (segment (start 141.605 94.74) (end 142.705 95.84) (width 0.2) (layer "F.Cu") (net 1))
 (segment (start 133.3675 78.985) (end 133.3675 86.3225) (width 0.2) (layer "F.Cu") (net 1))
 (segment (start 140.845 82.04) (end 141.5 82.04) (width 0.2) (layer "F.Cu") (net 1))
 (segment (start 138.905 84.124364) (end 140.989364 82.04) (width 0.2) (layer "F.Cu") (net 1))
 (segment (start 138.3725 82.04) (end 141.605 82.04) (width 0.2) (layer "F.Cu") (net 1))
 (segment (start 152.223226 108.185874) (end 142.350874 108.185874) (width 0.2) (layer "F.Cu") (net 1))
 (segment (start 134.3425 78.01) (end 133.3675 78.985) (width 0.2) (layer "F.Cu") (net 1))
 (segment (start 159.385 120.14) (end 158.285 119.04) (width 0.2) (layer "F.Cu") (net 1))
 (segment (start 154.8674 105.7026) (end 157.6476 105.7026) (width 0.2) (layer "F.Cu") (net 1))
 (segment (start 157.6476 105.7026) (end 159.385 107.44) (width 0.2) (layer "F.Cu") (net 1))
 (segment (start 141.605 120.14) (end 142.705 119.04) (width 0.2) (layer "F.Cu") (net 1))
 (segment (start 161.07 82.04) (end 159.385 82.04) (width 0.2) (layer "F.Cu") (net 1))
 (segment (start 133.3675 86.3225) (end 134.04 86.995) (width 0.2) (layer "F.Cu") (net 1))
 (segment (start 159.385 82.04) (end 162.3475 82.04) (width 0.2) (layer "F.Cu") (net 1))
 (segment (start 142.705 108.54) (end 141.605 107.44) (width 0.2) (layer "F.Cu") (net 1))
 (segment (start 142.350874 108.185874) (end 141.605 107.44) (width 0.2) (layer "F.Cu") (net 1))
 (segment (start 162.3475 82.04) (end 166.6475 77.74) (width 0.2) (layer "F.Cu") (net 1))
 (segment (start 140.989364 94.74) (end 138.905 92.655636) (width 0.2) (layer "F.Cu") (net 1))
 (segment (start 153.78 106.79) (end 154.8674 105.7026) (width 0.2) (layer "F.Cu") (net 1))
 (segment (start 142.705 119.04) (end 142.705 108.54) (width 0.2) (layer "F.Cu") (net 1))
 (segment (start 142.705 95.84) (end 142.705 106.34) (width 0.2) (layer "F.Cu") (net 1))
 (segment (start 134.3425 84.2725) (end 134.3425 80.01) (width 0.2) (layer "F.Cu") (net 4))
 (segment (start 136.115 86.045) (end 134.3425 84.2725) (width 0.2) (layer "F.Cu") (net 4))
 (segment (start 166.95 86.995) (end 166.6475 86.6925) (width 0.2) (layer "F.Cu") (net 3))
 (segment (start 166.6475 86.6925) (end 166.6475 79.74) (width 0.2) (layer "F.Cu") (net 3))
 (segment (start 135.89 88.17) (end 136.115 87.945) (width 0.2) (layer "F.Cu") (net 5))
 (segment (start 135.89 91.44) (end 135.89 88.17) (width 0.2) (layer "F.Cu") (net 5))
 (segment (start 165.1 88.17) (end 164.875 87.945) (width 0.2) (layer "F.Cu") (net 2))
 (segment (start 165.1 87.97) (end 165.075 87.945) (width 0.2) (layer "F.Cu") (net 2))
 (segment (start 165.1 91.44) (end 165.1 87.97) (width 0.2) (layer "F.Cu") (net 2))
 (segment (start 160.000636 104.9) (end 159.385 104.9) (width 0.2) (layer "F.Cu") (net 6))
 (segment (start 166.925 91.44) (end 166.925 97.975636) (width 0.2) (layer "F.Cu") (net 6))
 (segment (start 166.925 97.975636) (end 160.000636 104.9) (width 0.2) (layer "F.Cu") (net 6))
 (segment (start 140.989364 104.9) (end 141.605 104.9) (width 0.2) (layer "F.Cu") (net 7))
 (segment (start 134.065 97.975636) (end 140.989364 104.9) (width 0.2) (layer "F.Cu") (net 7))
 (segment (start 134.065 91.44) (end 134.065 97.975636) (width 0.2) (layer "F.Cu") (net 7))
 (segment (start 141.46 77) (end 141.5 76.96) (width 0.2) (layer "F.Cu") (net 8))
 (segment (start 140.884364 76.96) (end 141.5 76.96) (width 0.2) (layer "F.Cu") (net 8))
 (segment (start 139.9125 79.5) (end 141.5 79.5) (width 0.2) (layer "F.Cu") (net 9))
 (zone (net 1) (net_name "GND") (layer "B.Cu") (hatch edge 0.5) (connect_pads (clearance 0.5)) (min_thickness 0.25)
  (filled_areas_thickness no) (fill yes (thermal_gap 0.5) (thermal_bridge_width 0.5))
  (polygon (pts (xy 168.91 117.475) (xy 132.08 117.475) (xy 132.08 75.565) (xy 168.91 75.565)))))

